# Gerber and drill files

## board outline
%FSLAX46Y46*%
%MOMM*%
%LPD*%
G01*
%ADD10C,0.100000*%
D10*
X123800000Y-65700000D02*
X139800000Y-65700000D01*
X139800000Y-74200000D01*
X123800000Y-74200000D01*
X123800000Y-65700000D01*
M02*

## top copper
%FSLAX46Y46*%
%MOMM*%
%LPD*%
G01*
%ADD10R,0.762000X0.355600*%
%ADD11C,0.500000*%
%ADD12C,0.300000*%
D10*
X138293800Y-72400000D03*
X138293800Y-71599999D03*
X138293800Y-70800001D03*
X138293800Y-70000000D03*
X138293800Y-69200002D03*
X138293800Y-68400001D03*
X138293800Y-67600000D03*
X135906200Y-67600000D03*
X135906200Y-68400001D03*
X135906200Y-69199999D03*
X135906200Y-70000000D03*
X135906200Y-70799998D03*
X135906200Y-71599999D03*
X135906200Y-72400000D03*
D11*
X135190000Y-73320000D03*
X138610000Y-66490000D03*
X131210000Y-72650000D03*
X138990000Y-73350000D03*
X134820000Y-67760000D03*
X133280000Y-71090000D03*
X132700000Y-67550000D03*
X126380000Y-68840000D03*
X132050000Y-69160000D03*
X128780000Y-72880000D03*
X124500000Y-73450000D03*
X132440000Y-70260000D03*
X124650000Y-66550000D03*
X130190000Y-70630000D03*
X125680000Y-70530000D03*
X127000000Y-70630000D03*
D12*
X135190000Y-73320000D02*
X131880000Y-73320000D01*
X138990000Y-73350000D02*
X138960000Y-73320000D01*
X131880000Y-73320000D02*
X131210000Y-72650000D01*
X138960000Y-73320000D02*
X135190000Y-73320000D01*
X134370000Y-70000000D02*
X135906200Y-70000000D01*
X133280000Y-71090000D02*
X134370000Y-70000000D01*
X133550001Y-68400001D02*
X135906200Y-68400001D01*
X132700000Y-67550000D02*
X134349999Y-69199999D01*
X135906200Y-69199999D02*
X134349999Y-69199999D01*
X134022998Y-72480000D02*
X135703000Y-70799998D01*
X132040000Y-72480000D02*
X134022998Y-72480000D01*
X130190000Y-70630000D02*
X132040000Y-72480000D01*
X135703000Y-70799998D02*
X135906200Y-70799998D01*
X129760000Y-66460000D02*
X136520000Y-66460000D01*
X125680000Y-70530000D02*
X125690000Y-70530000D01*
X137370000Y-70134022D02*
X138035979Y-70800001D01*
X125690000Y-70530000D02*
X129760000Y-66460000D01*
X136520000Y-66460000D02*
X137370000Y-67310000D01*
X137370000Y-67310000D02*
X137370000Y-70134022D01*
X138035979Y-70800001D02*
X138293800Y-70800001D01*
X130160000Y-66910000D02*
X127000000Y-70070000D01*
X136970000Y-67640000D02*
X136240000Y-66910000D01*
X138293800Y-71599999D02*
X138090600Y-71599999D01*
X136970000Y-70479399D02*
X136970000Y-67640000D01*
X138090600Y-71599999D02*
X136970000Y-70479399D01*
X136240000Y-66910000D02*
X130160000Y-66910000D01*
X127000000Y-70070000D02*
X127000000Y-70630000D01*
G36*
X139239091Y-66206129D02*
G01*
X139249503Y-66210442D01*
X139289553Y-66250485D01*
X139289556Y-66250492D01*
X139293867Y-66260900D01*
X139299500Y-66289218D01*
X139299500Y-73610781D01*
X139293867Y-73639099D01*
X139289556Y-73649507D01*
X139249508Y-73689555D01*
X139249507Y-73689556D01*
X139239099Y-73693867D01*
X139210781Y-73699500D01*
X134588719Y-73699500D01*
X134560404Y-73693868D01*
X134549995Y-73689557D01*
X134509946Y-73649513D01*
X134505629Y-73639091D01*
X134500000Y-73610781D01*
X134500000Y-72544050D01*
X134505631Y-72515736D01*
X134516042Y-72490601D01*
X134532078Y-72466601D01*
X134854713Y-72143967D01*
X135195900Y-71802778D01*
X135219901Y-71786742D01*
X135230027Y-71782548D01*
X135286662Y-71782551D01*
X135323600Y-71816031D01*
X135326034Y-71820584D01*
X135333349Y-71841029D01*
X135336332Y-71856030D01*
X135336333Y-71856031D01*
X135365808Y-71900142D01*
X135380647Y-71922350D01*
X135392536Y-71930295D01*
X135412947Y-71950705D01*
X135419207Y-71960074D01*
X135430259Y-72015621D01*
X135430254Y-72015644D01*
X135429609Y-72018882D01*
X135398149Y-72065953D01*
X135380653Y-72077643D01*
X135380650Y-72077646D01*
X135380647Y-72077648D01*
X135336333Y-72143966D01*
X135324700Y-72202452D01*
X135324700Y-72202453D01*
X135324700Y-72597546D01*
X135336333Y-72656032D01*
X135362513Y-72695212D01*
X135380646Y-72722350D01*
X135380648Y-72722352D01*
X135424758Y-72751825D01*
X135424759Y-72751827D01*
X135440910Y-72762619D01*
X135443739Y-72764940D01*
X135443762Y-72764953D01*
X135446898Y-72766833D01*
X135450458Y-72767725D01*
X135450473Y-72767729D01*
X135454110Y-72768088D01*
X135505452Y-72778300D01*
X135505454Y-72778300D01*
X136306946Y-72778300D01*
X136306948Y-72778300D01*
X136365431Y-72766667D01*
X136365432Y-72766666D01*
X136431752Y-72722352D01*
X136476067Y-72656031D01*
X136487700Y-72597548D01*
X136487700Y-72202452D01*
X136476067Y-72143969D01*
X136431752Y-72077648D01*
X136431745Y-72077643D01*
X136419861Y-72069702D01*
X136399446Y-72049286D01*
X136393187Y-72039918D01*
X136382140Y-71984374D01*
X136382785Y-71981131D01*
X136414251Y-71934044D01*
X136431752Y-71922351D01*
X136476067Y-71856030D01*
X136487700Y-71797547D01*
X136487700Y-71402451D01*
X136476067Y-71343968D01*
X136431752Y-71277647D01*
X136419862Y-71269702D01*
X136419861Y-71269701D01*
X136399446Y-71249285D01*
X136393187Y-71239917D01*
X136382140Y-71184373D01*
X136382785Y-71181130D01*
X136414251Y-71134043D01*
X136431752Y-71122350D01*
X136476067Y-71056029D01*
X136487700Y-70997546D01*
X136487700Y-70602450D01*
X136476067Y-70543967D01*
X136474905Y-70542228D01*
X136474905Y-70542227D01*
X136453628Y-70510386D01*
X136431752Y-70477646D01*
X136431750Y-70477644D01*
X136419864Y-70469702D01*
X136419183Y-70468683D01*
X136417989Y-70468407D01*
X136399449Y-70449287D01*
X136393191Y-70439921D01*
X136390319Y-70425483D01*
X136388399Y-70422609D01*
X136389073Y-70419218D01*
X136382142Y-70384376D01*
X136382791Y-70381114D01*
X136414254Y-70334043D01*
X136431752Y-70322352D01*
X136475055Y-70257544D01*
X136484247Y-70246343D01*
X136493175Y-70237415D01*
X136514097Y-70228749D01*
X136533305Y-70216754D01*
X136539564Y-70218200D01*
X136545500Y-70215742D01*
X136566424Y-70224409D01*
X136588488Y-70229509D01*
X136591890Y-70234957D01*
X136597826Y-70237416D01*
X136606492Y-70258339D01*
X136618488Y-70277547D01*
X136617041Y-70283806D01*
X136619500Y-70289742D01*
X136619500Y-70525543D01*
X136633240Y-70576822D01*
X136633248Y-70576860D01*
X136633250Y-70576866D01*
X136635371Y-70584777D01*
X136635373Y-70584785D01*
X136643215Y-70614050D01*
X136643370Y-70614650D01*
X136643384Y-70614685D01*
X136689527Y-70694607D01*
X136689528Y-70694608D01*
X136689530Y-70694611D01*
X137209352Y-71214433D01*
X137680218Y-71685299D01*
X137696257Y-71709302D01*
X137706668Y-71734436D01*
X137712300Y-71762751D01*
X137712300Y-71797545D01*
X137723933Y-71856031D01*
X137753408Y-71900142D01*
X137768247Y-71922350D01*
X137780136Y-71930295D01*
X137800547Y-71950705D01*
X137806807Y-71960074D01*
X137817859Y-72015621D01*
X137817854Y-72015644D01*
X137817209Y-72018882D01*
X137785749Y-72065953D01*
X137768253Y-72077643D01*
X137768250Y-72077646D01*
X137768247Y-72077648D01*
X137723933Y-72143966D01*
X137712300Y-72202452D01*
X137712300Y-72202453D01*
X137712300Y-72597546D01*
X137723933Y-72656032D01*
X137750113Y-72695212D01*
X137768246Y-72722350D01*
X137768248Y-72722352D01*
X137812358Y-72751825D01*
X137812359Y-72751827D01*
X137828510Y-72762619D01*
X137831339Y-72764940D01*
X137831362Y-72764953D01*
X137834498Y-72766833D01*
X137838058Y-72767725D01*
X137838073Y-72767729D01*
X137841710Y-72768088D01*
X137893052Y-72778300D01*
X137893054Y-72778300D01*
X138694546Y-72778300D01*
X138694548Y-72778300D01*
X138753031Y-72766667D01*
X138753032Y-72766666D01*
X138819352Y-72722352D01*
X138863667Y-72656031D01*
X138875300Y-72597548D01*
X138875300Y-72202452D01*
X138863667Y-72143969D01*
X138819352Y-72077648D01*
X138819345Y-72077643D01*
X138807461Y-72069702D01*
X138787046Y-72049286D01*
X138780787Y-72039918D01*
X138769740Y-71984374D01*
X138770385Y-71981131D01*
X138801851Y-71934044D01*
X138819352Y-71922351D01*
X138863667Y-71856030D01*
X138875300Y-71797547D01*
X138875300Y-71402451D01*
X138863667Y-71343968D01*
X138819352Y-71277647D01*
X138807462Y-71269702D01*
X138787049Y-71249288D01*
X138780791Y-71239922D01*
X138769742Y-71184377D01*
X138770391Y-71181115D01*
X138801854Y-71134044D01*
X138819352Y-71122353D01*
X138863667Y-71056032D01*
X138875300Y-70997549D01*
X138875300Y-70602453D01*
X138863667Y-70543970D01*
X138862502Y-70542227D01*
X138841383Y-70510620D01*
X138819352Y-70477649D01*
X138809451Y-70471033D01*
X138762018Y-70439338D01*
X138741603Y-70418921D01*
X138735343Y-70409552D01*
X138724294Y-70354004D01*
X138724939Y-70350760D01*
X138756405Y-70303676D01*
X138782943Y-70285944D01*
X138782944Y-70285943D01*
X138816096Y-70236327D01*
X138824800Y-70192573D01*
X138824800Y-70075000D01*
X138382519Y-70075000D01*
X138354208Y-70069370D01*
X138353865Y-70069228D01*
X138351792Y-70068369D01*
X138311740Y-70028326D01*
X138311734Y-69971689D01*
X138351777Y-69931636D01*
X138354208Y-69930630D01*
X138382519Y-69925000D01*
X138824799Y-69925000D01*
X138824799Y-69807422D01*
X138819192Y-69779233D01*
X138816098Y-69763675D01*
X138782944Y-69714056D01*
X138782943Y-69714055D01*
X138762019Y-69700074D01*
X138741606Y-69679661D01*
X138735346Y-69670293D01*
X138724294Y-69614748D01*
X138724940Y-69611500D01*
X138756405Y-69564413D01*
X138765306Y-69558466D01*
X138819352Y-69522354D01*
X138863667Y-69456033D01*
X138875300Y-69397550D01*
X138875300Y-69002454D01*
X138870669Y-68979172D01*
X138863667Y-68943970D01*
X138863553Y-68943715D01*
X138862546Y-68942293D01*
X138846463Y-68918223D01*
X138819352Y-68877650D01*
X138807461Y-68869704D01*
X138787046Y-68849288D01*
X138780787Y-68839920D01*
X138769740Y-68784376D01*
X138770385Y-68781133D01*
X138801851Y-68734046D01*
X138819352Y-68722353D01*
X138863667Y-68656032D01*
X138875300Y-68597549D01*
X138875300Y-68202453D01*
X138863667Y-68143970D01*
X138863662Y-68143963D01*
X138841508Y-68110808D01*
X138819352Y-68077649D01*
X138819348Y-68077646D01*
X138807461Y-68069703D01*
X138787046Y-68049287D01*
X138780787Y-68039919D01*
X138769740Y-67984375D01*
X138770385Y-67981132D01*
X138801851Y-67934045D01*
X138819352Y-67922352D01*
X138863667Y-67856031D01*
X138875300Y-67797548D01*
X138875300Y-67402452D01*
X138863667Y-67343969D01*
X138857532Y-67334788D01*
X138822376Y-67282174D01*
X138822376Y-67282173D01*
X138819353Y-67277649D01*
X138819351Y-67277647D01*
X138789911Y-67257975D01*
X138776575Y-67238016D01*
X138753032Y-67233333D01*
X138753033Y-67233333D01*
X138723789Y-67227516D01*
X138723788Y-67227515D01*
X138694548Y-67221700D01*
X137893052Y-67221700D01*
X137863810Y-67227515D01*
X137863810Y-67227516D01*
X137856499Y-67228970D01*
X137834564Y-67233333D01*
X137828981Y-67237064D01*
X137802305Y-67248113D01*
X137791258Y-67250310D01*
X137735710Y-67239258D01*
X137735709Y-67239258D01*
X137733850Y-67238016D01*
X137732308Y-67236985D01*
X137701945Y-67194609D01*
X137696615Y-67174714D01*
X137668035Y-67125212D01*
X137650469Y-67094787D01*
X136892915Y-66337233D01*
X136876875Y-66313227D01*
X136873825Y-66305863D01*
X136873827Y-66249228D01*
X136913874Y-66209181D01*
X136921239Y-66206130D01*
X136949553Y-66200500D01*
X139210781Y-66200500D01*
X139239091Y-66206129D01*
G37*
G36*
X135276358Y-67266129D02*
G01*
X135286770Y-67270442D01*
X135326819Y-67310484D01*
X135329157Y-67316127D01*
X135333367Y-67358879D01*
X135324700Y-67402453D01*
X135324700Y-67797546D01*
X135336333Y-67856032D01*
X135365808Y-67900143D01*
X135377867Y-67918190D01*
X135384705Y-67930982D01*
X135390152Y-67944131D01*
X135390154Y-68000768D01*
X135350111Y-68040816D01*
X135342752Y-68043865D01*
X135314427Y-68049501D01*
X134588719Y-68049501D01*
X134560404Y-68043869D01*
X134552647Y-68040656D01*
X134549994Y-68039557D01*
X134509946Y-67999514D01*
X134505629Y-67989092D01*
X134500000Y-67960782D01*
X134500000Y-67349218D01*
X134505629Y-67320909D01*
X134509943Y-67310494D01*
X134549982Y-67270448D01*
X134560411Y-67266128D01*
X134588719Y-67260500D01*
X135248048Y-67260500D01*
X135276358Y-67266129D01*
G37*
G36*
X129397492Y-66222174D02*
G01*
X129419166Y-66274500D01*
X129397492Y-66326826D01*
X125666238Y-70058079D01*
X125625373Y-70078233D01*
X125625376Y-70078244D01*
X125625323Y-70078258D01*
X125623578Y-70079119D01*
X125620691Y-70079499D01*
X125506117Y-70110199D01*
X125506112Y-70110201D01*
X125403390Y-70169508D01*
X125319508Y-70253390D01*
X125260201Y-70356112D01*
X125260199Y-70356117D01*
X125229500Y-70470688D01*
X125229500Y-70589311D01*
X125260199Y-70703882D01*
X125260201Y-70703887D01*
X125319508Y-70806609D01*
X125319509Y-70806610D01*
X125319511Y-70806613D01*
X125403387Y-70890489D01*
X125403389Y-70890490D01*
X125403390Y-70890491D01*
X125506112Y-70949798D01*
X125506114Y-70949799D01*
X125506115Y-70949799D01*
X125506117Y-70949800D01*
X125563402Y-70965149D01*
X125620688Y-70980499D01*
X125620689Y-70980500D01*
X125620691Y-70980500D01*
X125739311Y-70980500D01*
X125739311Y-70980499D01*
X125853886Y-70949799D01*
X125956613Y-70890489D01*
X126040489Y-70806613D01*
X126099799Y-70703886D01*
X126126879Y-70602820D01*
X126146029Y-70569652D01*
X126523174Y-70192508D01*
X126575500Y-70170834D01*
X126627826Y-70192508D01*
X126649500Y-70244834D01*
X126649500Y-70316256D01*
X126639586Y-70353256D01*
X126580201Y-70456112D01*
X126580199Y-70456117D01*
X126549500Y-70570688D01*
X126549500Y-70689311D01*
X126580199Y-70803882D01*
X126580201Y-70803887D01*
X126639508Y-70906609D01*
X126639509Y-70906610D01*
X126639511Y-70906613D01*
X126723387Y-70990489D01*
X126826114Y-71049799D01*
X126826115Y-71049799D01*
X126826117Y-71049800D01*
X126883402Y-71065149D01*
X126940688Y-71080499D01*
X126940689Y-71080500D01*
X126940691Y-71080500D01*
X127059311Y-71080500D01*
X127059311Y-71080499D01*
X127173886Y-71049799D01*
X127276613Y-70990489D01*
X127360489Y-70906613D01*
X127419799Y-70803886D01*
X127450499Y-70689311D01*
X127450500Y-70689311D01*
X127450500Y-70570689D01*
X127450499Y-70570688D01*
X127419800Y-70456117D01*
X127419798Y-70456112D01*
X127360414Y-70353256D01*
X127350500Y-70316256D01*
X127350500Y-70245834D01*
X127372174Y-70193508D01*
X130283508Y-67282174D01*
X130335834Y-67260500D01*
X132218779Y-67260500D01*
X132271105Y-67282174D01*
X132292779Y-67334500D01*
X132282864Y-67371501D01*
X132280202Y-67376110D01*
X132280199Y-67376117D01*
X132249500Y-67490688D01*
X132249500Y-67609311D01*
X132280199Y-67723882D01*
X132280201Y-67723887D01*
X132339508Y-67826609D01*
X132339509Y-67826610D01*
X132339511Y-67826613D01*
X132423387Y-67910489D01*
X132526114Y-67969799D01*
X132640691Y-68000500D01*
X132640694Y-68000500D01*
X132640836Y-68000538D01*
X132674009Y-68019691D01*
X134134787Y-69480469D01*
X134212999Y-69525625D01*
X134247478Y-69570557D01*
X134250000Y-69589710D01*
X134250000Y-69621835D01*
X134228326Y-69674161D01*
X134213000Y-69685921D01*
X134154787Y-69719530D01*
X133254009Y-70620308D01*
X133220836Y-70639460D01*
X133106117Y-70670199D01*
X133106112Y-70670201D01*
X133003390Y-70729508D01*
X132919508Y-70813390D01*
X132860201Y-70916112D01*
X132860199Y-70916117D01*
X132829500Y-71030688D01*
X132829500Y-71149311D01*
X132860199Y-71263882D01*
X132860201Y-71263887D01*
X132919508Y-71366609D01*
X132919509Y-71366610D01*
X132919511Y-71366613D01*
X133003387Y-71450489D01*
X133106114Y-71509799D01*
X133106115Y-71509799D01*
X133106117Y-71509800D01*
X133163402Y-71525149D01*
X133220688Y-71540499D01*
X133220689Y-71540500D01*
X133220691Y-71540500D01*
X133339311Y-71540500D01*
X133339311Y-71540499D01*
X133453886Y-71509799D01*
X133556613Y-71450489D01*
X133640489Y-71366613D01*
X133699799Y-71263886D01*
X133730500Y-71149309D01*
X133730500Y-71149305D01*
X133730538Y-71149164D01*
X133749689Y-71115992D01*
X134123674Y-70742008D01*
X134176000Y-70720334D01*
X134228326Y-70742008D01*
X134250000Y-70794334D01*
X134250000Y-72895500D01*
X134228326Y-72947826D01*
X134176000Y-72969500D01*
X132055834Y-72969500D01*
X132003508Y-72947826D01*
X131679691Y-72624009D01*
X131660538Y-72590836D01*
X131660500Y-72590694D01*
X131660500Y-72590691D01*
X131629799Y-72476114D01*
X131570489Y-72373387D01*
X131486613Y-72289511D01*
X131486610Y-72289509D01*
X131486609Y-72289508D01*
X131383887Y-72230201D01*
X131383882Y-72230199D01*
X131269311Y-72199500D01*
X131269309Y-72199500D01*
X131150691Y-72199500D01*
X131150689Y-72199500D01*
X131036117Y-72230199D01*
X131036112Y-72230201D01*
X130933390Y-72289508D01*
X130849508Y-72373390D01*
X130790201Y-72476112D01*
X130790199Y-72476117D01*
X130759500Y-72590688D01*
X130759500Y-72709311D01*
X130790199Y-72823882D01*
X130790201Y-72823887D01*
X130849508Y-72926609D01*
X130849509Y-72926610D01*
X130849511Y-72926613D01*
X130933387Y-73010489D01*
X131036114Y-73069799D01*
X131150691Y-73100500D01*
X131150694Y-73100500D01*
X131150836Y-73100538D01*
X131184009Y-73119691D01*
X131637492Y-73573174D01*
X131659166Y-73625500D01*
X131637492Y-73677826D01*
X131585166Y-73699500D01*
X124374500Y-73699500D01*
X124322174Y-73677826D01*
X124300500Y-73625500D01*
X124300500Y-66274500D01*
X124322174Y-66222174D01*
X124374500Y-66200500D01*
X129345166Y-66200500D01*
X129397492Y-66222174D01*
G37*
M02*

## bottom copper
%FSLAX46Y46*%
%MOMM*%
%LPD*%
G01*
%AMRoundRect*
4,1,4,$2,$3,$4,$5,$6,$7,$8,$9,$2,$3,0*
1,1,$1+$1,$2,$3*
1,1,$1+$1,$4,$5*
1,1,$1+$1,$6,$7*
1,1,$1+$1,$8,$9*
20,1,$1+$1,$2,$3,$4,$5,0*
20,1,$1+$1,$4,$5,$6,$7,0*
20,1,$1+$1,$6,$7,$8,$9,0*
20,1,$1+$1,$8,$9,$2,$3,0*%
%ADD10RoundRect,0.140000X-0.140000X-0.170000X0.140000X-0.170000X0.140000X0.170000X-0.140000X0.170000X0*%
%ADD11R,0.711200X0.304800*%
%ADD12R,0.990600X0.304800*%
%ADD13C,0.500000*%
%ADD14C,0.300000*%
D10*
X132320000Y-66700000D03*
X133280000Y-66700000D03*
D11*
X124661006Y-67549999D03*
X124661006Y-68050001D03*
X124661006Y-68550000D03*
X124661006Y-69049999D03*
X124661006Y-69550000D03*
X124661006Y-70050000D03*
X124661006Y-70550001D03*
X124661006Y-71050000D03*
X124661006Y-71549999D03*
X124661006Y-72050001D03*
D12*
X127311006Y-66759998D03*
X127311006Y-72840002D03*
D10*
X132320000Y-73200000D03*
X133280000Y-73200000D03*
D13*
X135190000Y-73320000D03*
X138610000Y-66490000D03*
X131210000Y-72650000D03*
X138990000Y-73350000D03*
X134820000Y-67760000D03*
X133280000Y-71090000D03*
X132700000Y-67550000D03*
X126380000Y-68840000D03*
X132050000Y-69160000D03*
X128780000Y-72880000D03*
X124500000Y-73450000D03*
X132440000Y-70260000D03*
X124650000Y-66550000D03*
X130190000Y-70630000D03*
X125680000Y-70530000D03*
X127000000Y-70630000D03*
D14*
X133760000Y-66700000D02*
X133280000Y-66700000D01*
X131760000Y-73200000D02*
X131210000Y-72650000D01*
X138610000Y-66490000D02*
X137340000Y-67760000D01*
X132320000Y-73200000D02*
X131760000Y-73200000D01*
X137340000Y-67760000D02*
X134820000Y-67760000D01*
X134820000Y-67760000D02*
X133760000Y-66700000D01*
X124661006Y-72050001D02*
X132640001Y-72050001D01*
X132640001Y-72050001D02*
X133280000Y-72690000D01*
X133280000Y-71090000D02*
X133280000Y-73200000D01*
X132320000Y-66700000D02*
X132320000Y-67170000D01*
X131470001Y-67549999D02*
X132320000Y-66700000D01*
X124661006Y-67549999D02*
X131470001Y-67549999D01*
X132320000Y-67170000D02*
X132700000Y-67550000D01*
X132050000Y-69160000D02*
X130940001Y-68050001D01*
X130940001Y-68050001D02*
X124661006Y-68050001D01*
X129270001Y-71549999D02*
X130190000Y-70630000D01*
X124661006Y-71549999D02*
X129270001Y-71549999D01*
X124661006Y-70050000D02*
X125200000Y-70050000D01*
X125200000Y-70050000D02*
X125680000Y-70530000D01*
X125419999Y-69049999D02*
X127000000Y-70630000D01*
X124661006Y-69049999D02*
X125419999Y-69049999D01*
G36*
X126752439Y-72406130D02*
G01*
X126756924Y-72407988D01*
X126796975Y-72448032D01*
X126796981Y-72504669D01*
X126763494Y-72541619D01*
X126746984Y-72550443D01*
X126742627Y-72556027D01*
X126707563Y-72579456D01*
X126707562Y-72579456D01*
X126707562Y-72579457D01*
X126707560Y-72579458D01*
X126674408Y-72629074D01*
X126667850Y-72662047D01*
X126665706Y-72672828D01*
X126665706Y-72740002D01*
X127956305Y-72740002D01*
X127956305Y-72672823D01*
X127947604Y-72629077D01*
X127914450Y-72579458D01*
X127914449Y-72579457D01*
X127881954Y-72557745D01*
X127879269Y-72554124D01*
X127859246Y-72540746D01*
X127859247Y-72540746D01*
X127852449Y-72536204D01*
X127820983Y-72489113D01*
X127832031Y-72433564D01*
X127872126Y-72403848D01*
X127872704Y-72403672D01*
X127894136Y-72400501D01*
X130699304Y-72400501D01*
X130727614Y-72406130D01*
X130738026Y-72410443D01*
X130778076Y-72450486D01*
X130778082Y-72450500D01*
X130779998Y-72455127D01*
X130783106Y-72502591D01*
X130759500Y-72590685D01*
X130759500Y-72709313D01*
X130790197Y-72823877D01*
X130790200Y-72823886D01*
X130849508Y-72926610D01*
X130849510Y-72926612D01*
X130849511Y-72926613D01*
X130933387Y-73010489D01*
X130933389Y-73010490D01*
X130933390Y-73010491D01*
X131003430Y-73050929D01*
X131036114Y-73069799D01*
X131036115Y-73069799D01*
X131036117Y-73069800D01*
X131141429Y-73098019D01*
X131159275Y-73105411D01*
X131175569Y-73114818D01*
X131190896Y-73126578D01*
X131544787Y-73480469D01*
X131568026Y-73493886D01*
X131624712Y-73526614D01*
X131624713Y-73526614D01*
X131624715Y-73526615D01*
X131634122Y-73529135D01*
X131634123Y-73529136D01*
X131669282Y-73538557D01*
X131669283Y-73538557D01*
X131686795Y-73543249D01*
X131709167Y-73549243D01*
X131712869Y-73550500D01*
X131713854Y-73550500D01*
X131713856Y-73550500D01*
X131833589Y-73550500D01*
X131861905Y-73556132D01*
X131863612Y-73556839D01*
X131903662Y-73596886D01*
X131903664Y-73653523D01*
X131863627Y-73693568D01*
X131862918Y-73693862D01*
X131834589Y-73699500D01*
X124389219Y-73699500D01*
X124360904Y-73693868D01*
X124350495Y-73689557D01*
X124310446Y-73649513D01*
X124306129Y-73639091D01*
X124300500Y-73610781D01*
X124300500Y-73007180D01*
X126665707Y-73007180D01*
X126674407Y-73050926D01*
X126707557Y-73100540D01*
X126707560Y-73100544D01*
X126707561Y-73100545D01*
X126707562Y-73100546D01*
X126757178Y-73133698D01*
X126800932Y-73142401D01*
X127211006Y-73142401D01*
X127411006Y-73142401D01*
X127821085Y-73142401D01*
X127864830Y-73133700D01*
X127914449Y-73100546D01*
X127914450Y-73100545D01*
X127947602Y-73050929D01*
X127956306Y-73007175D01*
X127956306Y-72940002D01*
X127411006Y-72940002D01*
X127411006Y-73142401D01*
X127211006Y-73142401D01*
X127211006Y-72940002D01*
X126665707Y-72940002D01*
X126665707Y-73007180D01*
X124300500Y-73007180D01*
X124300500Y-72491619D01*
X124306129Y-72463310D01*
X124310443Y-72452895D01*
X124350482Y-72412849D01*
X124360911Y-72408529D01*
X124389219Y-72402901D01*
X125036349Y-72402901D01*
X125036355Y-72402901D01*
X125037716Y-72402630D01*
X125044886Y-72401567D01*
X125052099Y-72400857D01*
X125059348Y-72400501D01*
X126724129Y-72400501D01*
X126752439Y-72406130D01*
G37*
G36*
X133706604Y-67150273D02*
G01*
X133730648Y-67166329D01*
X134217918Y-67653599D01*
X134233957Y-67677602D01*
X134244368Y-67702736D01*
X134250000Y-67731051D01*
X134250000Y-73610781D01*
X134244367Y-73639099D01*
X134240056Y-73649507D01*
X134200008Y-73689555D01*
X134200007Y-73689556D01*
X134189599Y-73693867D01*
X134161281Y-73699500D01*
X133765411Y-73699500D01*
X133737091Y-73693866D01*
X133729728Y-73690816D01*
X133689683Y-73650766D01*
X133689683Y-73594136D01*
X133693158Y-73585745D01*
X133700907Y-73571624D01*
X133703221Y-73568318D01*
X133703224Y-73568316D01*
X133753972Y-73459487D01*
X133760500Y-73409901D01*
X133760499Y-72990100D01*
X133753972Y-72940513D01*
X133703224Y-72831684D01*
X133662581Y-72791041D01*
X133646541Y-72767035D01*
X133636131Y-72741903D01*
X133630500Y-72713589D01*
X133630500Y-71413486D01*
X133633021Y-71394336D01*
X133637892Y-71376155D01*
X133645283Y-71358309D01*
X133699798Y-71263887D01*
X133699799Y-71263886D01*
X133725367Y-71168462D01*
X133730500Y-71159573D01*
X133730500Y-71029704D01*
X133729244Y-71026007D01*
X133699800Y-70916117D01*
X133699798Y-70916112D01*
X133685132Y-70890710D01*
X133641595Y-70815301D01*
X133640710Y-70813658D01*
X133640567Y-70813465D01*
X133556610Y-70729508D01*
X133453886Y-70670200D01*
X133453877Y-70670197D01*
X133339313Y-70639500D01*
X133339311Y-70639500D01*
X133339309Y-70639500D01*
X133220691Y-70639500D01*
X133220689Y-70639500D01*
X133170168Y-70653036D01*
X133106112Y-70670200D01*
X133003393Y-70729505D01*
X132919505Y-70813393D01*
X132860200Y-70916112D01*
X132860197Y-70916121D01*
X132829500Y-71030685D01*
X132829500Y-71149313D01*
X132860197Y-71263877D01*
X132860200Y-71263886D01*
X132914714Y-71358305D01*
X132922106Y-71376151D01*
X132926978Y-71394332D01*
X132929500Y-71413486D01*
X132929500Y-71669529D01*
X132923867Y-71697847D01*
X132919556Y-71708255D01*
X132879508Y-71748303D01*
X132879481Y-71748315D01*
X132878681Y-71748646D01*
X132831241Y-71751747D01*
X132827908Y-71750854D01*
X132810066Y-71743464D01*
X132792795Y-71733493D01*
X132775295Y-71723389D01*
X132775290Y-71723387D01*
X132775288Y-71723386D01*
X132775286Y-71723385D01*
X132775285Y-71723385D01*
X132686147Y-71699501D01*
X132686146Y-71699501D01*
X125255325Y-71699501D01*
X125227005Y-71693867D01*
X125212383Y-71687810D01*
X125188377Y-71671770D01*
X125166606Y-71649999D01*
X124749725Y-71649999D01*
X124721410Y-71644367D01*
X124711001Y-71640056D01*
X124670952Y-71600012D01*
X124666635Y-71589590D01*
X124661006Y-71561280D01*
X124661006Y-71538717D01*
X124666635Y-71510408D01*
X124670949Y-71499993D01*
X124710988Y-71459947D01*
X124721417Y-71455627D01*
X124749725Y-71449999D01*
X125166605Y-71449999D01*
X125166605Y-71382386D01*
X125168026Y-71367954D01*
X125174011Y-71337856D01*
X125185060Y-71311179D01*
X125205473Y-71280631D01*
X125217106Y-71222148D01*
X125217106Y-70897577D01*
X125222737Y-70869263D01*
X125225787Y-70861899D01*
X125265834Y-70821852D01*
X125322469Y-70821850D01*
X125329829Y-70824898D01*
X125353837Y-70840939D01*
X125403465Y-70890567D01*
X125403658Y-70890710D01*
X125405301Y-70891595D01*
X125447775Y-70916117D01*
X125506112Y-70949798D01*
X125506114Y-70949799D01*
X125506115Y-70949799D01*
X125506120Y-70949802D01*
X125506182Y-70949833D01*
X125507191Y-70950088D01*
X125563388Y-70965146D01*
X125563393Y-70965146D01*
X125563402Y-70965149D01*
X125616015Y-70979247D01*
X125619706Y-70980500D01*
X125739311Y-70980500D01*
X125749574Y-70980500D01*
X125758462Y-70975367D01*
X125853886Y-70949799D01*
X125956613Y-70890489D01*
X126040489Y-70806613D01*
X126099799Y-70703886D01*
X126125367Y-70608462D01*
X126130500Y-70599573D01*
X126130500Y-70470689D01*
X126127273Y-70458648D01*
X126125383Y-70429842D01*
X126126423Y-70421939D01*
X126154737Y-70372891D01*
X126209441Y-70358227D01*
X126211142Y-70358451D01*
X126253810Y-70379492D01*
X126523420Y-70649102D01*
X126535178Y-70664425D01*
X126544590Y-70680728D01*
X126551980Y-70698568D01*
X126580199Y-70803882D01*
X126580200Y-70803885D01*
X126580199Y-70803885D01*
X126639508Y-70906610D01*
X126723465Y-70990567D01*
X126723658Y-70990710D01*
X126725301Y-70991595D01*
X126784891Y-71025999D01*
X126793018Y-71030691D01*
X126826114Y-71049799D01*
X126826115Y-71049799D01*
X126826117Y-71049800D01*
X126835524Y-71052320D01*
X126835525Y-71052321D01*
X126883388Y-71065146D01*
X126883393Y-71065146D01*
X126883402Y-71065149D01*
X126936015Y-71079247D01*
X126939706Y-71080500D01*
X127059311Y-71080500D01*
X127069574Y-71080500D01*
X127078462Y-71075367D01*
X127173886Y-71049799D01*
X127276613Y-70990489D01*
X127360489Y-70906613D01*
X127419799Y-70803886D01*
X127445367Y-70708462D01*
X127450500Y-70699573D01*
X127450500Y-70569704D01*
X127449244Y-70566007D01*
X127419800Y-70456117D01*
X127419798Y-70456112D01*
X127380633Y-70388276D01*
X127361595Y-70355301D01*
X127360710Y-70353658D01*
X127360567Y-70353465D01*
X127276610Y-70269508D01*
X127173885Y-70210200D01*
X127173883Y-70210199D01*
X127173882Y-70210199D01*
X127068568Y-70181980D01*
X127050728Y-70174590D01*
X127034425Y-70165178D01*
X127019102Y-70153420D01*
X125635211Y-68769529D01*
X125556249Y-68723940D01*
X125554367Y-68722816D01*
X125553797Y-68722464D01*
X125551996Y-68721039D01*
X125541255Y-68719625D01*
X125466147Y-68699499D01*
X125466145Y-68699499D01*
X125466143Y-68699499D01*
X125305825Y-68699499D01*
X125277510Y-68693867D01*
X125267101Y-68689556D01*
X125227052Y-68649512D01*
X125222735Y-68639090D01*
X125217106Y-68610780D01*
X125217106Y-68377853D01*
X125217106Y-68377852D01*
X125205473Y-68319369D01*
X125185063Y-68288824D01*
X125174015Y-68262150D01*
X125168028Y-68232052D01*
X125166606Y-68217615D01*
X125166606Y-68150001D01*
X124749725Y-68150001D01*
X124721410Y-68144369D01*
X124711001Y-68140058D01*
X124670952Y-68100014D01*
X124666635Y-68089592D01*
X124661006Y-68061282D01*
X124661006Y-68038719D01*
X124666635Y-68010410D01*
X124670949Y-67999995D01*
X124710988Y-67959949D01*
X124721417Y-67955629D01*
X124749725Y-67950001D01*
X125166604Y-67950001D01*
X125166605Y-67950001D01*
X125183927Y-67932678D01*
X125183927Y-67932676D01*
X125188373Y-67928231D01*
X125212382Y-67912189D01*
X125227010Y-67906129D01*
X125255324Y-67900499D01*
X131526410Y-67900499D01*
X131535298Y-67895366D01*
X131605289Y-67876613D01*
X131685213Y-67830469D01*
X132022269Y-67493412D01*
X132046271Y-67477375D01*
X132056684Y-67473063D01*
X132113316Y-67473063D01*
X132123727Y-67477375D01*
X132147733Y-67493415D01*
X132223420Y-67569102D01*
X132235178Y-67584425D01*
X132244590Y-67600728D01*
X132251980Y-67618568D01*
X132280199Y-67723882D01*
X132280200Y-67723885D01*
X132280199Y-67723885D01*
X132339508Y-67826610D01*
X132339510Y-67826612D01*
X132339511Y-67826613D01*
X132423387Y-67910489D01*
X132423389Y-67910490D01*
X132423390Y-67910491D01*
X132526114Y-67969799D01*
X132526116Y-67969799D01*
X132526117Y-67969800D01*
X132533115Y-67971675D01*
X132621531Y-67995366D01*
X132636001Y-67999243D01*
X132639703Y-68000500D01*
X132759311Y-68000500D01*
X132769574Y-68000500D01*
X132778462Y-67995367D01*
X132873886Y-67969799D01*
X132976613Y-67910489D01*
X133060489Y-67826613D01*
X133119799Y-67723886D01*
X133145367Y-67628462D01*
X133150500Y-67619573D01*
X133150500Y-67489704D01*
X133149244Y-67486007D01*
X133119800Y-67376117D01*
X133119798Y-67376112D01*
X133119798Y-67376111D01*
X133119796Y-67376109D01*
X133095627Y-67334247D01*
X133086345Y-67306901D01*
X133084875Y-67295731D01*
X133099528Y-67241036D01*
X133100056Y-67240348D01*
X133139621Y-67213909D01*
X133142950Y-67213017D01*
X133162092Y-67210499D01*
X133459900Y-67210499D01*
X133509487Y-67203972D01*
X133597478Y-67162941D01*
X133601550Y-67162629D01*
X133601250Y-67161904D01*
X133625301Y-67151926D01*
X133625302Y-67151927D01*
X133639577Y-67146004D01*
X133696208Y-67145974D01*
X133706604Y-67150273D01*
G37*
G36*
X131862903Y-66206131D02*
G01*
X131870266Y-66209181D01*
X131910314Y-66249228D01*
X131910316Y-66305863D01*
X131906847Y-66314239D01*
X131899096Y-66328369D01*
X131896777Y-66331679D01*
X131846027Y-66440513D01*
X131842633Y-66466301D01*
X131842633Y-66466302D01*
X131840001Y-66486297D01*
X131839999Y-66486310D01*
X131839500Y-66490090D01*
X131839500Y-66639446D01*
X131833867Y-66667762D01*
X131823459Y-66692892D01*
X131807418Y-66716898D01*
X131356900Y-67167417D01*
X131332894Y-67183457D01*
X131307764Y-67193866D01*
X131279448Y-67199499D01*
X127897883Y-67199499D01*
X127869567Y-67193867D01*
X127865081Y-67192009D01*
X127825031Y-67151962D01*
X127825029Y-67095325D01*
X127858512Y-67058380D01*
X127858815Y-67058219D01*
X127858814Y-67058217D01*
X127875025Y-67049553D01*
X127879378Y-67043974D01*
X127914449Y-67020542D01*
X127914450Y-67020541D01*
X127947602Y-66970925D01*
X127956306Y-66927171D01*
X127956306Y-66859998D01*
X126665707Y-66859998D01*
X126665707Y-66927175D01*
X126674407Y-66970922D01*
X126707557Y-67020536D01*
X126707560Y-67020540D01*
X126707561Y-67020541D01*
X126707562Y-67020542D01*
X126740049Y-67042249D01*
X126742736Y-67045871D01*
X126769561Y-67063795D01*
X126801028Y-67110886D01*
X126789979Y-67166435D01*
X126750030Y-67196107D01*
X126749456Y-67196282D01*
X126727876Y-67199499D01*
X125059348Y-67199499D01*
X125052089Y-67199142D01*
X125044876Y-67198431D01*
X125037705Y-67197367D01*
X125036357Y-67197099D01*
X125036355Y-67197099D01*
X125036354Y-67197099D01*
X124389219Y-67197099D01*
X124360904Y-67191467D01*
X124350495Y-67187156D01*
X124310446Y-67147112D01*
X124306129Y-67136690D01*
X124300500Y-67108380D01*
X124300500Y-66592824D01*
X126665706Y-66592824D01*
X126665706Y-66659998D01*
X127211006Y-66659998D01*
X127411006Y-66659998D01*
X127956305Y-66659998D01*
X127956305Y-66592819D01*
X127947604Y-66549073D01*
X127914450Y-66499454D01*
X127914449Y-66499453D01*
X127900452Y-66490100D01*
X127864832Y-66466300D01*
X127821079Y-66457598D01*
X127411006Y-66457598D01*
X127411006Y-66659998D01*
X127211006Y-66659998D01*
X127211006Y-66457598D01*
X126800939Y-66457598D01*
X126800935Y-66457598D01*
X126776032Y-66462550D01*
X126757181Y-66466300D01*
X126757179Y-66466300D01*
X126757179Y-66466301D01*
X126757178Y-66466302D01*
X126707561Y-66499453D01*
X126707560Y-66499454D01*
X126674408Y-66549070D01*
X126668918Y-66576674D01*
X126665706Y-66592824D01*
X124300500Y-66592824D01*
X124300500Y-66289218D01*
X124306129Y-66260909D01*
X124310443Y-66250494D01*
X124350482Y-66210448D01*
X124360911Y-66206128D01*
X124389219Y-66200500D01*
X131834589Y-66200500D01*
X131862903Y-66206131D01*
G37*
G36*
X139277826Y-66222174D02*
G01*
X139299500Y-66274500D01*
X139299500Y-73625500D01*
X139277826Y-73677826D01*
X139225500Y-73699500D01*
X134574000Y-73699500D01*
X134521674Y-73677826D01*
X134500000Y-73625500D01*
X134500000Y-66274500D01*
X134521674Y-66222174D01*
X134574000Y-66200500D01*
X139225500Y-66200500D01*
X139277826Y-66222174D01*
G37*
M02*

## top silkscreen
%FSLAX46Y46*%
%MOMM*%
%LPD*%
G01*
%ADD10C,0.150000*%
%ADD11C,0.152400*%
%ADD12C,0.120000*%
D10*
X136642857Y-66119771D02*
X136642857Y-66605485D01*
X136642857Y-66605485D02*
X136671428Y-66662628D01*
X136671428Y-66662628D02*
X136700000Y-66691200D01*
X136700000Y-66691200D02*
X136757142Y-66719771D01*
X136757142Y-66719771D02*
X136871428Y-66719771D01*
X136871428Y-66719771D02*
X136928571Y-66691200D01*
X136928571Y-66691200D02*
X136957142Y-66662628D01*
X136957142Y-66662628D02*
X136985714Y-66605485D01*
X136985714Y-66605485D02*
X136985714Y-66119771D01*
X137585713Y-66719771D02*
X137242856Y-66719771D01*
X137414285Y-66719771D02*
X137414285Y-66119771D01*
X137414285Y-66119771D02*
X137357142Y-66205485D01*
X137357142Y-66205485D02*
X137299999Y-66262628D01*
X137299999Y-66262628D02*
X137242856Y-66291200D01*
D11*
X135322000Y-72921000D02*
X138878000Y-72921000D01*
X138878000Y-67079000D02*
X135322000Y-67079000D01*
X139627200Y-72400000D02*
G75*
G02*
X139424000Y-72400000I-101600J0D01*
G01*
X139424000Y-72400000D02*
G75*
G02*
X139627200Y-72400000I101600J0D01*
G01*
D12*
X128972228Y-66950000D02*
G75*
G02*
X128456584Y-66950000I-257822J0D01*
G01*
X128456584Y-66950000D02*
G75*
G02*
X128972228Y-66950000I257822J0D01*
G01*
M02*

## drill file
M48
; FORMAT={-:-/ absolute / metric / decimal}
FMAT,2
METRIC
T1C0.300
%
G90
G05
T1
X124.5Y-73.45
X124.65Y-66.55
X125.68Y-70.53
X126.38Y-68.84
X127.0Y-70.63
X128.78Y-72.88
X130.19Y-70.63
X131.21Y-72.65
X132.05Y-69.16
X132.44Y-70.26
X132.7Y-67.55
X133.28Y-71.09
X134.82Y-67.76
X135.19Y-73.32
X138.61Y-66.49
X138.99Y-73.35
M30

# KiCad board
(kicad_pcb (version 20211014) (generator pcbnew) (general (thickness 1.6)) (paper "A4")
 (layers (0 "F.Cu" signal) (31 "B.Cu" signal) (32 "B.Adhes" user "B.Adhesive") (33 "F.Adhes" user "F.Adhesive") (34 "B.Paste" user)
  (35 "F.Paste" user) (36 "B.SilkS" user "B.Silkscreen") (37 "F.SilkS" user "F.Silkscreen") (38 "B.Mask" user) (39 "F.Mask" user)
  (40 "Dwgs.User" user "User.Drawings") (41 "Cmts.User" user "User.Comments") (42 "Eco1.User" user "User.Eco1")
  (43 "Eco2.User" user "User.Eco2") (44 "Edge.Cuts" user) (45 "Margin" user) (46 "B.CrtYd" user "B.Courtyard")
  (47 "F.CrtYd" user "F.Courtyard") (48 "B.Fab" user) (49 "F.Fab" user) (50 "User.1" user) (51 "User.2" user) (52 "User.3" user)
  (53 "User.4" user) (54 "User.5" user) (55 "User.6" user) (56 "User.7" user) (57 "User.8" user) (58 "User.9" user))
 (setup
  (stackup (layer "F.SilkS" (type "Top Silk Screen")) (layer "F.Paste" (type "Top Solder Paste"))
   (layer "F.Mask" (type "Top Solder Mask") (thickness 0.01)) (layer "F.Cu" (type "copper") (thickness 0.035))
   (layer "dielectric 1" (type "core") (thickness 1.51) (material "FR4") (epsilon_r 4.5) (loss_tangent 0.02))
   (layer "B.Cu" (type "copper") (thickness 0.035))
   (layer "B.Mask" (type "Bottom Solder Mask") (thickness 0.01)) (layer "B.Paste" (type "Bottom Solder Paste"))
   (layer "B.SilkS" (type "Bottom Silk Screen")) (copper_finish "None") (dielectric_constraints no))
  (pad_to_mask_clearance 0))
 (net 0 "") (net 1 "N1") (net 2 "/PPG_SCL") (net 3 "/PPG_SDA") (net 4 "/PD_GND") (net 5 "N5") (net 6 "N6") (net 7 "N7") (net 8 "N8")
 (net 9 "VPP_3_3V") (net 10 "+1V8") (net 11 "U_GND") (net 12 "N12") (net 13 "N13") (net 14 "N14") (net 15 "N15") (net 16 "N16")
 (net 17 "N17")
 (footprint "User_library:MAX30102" (layer "F.Cu") (at 137.1 70 180)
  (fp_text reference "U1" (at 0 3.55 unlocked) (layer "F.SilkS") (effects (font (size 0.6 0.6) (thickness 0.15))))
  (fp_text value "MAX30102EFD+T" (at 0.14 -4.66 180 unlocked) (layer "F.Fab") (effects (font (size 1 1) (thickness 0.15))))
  (fp_line (start 1.778 -2.921) (end -1.778 -2.921) (layer "F.SilkS") (width 0.1524))
  (fp_line (start -1.778 2.921) (end 1.778 2.921) (layer "F.SilkS") (width 0.1524))
  (fp_circle (center -2.4256 -2.4) (end -2.324 -2.4) (layer "F.SilkS") (width 0.1524) (fill none))
  (pad "1" smd rect (at -1.1938 -2.4 180) (size 0.762 0.3556) (layers "F.Cu" "F.Paste" "F.Mask") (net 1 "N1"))
  (pad "2" smd rect (at -1.1938 -1.599999 180) (size 0.762 0.3556) (layers "F.Cu" "F.Paste" "F.Mask") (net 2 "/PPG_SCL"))
  (pad "3" smd rect (at -1.1938 -0.800001 180) (size 0.762 0.3556) (layers "F.Cu" "F.Paste" "F.Mask") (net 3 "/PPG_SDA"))
  (pad "4" smd rect (at -1.1938 0 180) (size 0.762 0.3556) (layers "F.Cu" "F.Paste" "F.Mask") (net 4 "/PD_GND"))
  (pad "5" smd rect (at -1.1938 0.799998 180) (size 0.762 0.3556) (layers "F.Cu" "F.Paste" "F.Mask") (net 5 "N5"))
  (pad "6" smd rect (at -1.1938 1.599999 180) (size 0.762 0.3556) (layers "F.Cu" "F.Paste" "F.Mask") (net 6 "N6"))
  (pad "7" smd rect (at -1.1938 2.4 180) (size 0.762 0.3556) (layers "F.Cu" "F.Paste" "F.Mask") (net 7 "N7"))
  (pad "8" smd rect (at 1.1938 2.4 180) (size 0.762 0.3556) (layers "F.Cu" "F.Paste" "F.Mask") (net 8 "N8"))
  (pad "9" smd rect (at 1.1938 1.599999 180) (size 0.762 0.3556) (layers "F.Cu" "F.Paste" "F.Mask") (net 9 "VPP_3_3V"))
  (pad "10" smd rect (at 1.1938 0.800001 180) (size 0.762 0.3556) (layers "F.Cu" "F.Paste" "F.Mask") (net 9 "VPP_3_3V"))
  (pad "11" smd rect (at 1.1938 0 180) (size 0.762 0.3556) (layers "F.Cu" "F.Paste" "F.Mask") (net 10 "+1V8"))
  (pad "12" smd rect (at 1.1938 -0.799998 180) (size 0.762 0.3556) (layers "F.Cu" "F.Paste" "F.Mask") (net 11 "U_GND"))
  (pad "13" smd rect (at 1.1938 -1.599999 180) (size 0.762 0.3556) (layers "F.Cu" "F.Paste" "F.Mask") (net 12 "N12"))
  (pad "14" smd rect (at 1.1938 -2.4 180) (size 0.762 0.3556) (layers "F.Cu" "F.Paste" "F.Mask") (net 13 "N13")))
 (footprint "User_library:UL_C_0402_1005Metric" (layer "B.Cu") (at 132.8 66.7)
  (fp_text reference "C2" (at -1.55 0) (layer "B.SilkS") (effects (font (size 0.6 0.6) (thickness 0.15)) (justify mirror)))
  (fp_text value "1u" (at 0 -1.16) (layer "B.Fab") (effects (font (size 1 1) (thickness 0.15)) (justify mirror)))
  (pad "1" smd roundrect locked (at -0.48 0) (size 0.56 0.62) (layers "B.Cu" "B.Paste" "B.Mask") (roundrect_rratio 0.25) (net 9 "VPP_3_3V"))
  (pad "2" smd roundrect locked (at 0.48 0) (size 0.56 0.62) (layers "B.Cu" "B.Paste" "B.Mask") (roundrect_rratio 0.25) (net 4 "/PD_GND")))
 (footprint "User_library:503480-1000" (layer "B.Cu") (at 126.164406 69.8 -90)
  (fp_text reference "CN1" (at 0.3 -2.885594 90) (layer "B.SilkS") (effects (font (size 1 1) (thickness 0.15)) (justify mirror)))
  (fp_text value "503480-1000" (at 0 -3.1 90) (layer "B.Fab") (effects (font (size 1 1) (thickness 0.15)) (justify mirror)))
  (fp_circle (center -2.85 -2.55) (end -2.5922 -2.5534) (layer "F.SilkS") (width 0.12) (fill none))
  (pad "1" smd rect (at -2.250001 1.5034 270) (size 0.3048 0.7112) (layers "B.Cu" "B.Paste" "B.Mask") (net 9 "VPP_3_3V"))
  (pad "2" smd rect (at -1.749999 1.5034 270) (size 0.3048 0.7112) (layers "B.Cu" "B.Paste" "B.Mask") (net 11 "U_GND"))
  (pad "3" smd rect (at -1.25 1.5034 270) (size 0.3048 0.7112) (layers "B.Cu" "B.Paste" "B.Mask") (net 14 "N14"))
  (pad "4" smd rect (at -0.750001 1.5034 270) (size 0.3048 0.7112) (layers "B.Cu" "B.Paste" "B.Mask") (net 2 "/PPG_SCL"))
  (pad "5" smd rect (at -0.25 1.5034 270) (size 0.3048 0.7112) (layers "B.Cu" "B.Paste" "B.Mask") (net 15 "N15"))
  (pad "6" smd rect (at 0.25 1.5034 270) (size 0.3048 0.7112) (layers "B.Cu" "B.Paste" "B.Mask") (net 3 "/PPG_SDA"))
  (pad "7" smd rect (at 0.750001 1.5034 270) (size 0.3048 0.7112) (layers "B.Cu" "B.Paste" "B.Mask") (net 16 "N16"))
  (pad "8" smd rect (at 1.25 1.5034 270) (size 0.3048 0.7112) (layers "B.Cu" "B.Paste" "B.Mask") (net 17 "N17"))
  (pad "9" smd rect (at 1.749999 1.5034 270) (size 0.3048 0.7112) (layers "B.Cu" "B.Paste" "B.Mask") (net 11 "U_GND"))
  (pad "10" smd rect (at 2.250001 1.5034 270) (size 0.3048 0.7112) (layers "B.Cu" "B.Paste" "B.Mask") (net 10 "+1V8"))
  (pad "11" smd rect (at -3.040002 -1.1466 270) (size 0.3048 0.9906) (layers "B.Cu" "B.Paste" "B.Mask") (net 11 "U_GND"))
  (pad "12" smd rect (at 3.040002 -1.1466 270) (size 0.3048 0.9906) (layers "B.Cu" "B.Paste" "B.Mask") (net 11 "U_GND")))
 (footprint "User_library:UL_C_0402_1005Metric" (layer "B.Cu") (at 132.8 73.2)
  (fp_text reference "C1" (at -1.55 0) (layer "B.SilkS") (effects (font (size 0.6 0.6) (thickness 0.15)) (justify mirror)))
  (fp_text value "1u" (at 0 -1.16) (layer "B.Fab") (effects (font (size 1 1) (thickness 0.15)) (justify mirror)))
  (pad "1" smd roundrect locked (at -0.48 0) (size 0.56 0.62) (layers "B.Cu" "B.Paste" "B.Mask") (roundrect_rratio 0.25) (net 4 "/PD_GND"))
  (pad "2" smd roundrect locked (at 0.48 0) (size 0.56 0.62) (layers "B.Cu" "B.Paste" "B.Mask") (roundrect_rratio 0.25) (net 10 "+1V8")))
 (gr_rect (start 123.8 65.7) (end 139.8 74.2) (layer "Edge.Cuts") (width 0.1) (fill none))
 (segment (start 135.19 73.32) (end 131.88 73.32) (width 0.3) (layer "F.Cu") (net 4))
 (segment (start 138.99 73.35) (end 138.96 73.32) (width 0.3) (layer "F.Cu") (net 4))
 (segment (start 131.88 73.32) (end 131.21 72.65) (width 0.3) (layer "F.Cu") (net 4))
 (segment (start 138.96 73.32) (end 135.19 73.32) (width 0.3) (layer "F.Cu") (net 4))
 (via (at 135.19 73.32) (size 0.5) (drill 0.3) (layers "F.Cu" "B.Cu") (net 4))
 (via (at 138.61 66.49) (size 0.5) (drill 0.3) (layers "F.Cu" "B.Cu") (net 4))
 (via (at 131.21 72.65) (size 0.5) (drill 0.3) (layers "F.Cu" "B.Cu") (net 4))
 (via (at 138.99 73.35) (size 0.5) (drill 0.3) (layers "F.Cu" "B.Cu") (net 4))
 (via (at 134.82 67.76) (size 0.5) (drill 0.3) (layers "F.Cu" "B.Cu") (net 4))
 (segment (start 133.76 66.7) (end 133.28 66.7) (width 0.3) (layer "B.Cu") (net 4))
 (segment (start 131.76 73.2) (end 131.21 72.65) (width 0.3) (layer "B.Cu") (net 4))
 (segment (start 138.61 66.49) (end 137.34 67.76) (width 0.3) (layer "B.Cu") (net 4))
 (segment (start 132.32 73.2) (end 131.76 73.2) (width 0.3) (layer "B.Cu") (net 4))
 (segment (start 137.34 67.76) (end 134.82 67.76) (width 0.3) (layer "B.Cu") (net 4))
 (segment (start 134.82 67.76) (end 133.76 66.7) (width 0.3) (layer "B.Cu") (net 4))
 (segment (start 134.37 70) (end 135.9062 70) (width 0.3) (layer "F.Cu") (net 10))
 (segment (start 133.28 71.09) (end 134.37 70) (width 0.3) (layer "F.Cu") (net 10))
 (via (at 133.28 71.09) (size 0.5) (drill 0.3) (layers "F.Cu" "B.Cu") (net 10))
 (segment (start 124.661006 72.050001) (end 132.640001 72.050001) (width 0.3) (layer "B.Cu") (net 10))
 (segment (start 132.640001 72.050001) (end 133.28 72.69) (width 0.3) (layer "B.Cu") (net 10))
 (segment (start 133.28 71.09) (end 133.28 73.2) (width 0.3) (layer "B.Cu") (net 10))
 (segment (start 133.550001 68.400001) (end 135.9062 68.400001) (width 0.3) (layer "F.Cu") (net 9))
 (segment (start 132.7 67.55) (end 134.349999 69.199999) (width 0.3) (layer "F.Cu") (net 9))
 (segment (start 135.9062 69.199999) (end 134.349999 69.199999) (width 0.3) (layer "F.Cu") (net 9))
 (via (at 132.7 67.55) (size 0.5) (drill 0.3) (layers "F.Cu" "B.Cu") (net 9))
 (segment (start 132.32 66.7) (end 132.32 67.17) (width 0.3) (layer "B.Cu") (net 9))
 (segment (start 131.470001 67.549999) (end 132.32 66.7) (width 0.3) (layer "B.Cu") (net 9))
 (segment (start 124.661006 67.549999) (end 131.470001 67.549999) (width 0.3) (layer "B.Cu") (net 9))
 (segment (start 132.32 67.17) (end 132.7 67.55) (width 0.3) (layer "B.Cu") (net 9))
 (segment (start 134.022998 72.48) (end 135.703 70.799998) (width 0.3) (layer "F.Cu") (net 11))
 (segment (start 132.04 72.48) (end 134.022998 72.48) (width 0.3) (layer "F.Cu") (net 11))
 (segment (start 130.19 70.63) (end 132.04 72.48) (width 0.3) (layer "F.Cu") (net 11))
 (segment (start 135.703 70.799998) (end 135.9062 70.799998) (width 0.3) (layer "F.Cu") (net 11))
 (via (at 126.38 68.84) (size 0.5) (drill 0.3) (layers "F.Cu" "B.Cu") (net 11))
 (via (at 132.05 69.16) (size 0.5) (drill 0.3) (layers "F.Cu" "B.Cu") (free) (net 11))
 (via (at 128.78 72.88) (size 0.5) (drill 0.3) (layers "F.Cu" "B.Cu") (free) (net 11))
 (via (at 124.5 73.45) (size 0.5) (drill 0.3) (layers "F.Cu" "B.Cu") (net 11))
 (via (at 132.44 70.26) (size 0.5) (drill 0.3) (layers "F.Cu" "B.Cu") (free) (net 11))
 (via (at 124.65 66.55) (size 0.5) (drill 0.3) (layers "F.Cu" "B.Cu") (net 11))
 (via (at 130.19 70.63) (size 0.5) (drill 0.3) (layers "F.Cu" "B.Cu") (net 11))
 (segment (start 132.05 69.16) (end 130.940001 68.050001) (width 0.3) (layer "B.Cu") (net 11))
 (segment (start 130.940001 68.050001) (end 124.661006 68.050001) (width 0.3) (layer "B.Cu") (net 11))
 (segment (start 129.270001 71.549999) (end 130.19 70.63) (width 0.3) (layer "B.Cu") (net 11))
 (segment (start 124.661006 71.549999) (end 129.270001 71.549999) (width 0.3) (layer "B.Cu") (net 11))
 (segment (start 129.76 66.46) (end 136.52 66.46) (width 0.3) (layer "F.Cu") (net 3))
 (segment (start 125.68 70.53) (end 125.69 70.53) (width 0.3) (layer "F.Cu") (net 3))
 (segment (start 137.37 70.134022) (end 138.035979 70.800001) (width 0.3) (layer "F.Cu") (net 3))
 (segment (start 125.69 70.53) (end 129.76 66.46) (width 0.3) (layer "F.Cu") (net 3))
 (segment (start 136.52 66.46) (end 137.37 67.31) (width 0.3) (layer "F.Cu") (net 3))
 (segment (start 137.37 67.31) (end 137.37 70.134022) (width 0.3) (layer "F.Cu") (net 3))
 (segment (start 138.035979 70.800001) (end 138.2938 70.800001) (width 0.3) (layer "F.Cu") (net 3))
 (via (at 125.68 70.53) (size 0.5) (drill 0.3) (layers "F.Cu" "B.Cu") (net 3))
 (segment (start 124.661006 70.05) (end 125.2 70.05) (width 0.3) (layer "B.Cu") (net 3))
 (segment (start 125.2 70.05) (end 125.68 70.53) (width 0.3) (layer "B.Cu") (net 3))
 (segment (start 130.16 66.91) (end 127 70.07) (width 0.3) (layer "F.Cu") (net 2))
 (segment (start 136.97 67.64) (end 136.24 66.91) (width 0.3) (layer "F.Cu") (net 2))
 (segment (start 138.2938 71.599999) (end 138.0906 71.599999) (width 0.3) (layer "F.Cu") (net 2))
 (segment (start 136.97 70.479399) (end 136.97 67.64) (width 0.3) (layer "F.Cu") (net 2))
 (segment (start 138.0906 71.599999) (end 136.97 70.479399) (width 0.3) (layer "F.Cu") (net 2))
 (segment (start 136.24 66.91) (end 130.16 66.91) (width 0.3) (layer "F.Cu") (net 2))
 (segment (start 127 70.07) (end 127 70.63) (width 0.3) (layer "F.Cu") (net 2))
 (via (at 127 70.63) (size 0.5) (drill 0.3) (layers "F.Cu" "B.Cu") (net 2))
 (segment (start 125.419999 69.049999) (end 127 70.63) (width 0.3) (layer "B.Cu") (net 2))
 (segment (start 124.661006 69.049999) (end 125.419999 69.049999) (width 0.3) (layer "B.Cu") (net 2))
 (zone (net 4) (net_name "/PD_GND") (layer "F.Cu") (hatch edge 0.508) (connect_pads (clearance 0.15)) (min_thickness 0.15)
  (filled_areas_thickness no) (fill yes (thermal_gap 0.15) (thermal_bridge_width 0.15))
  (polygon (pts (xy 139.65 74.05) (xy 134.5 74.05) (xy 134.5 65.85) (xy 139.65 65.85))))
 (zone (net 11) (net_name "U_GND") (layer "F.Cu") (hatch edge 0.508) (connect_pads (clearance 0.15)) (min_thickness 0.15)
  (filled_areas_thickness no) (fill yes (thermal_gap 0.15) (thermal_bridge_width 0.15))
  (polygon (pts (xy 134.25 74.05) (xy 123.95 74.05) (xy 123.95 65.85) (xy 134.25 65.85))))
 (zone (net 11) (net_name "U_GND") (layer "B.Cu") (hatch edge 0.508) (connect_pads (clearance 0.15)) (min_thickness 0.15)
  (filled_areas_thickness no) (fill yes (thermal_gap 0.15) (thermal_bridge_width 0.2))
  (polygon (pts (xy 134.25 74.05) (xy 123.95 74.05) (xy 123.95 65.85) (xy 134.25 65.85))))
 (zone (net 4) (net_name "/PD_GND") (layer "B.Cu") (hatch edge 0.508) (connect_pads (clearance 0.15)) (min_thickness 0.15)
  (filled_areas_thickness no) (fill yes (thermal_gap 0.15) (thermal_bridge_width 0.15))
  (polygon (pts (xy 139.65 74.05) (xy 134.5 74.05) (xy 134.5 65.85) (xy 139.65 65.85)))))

